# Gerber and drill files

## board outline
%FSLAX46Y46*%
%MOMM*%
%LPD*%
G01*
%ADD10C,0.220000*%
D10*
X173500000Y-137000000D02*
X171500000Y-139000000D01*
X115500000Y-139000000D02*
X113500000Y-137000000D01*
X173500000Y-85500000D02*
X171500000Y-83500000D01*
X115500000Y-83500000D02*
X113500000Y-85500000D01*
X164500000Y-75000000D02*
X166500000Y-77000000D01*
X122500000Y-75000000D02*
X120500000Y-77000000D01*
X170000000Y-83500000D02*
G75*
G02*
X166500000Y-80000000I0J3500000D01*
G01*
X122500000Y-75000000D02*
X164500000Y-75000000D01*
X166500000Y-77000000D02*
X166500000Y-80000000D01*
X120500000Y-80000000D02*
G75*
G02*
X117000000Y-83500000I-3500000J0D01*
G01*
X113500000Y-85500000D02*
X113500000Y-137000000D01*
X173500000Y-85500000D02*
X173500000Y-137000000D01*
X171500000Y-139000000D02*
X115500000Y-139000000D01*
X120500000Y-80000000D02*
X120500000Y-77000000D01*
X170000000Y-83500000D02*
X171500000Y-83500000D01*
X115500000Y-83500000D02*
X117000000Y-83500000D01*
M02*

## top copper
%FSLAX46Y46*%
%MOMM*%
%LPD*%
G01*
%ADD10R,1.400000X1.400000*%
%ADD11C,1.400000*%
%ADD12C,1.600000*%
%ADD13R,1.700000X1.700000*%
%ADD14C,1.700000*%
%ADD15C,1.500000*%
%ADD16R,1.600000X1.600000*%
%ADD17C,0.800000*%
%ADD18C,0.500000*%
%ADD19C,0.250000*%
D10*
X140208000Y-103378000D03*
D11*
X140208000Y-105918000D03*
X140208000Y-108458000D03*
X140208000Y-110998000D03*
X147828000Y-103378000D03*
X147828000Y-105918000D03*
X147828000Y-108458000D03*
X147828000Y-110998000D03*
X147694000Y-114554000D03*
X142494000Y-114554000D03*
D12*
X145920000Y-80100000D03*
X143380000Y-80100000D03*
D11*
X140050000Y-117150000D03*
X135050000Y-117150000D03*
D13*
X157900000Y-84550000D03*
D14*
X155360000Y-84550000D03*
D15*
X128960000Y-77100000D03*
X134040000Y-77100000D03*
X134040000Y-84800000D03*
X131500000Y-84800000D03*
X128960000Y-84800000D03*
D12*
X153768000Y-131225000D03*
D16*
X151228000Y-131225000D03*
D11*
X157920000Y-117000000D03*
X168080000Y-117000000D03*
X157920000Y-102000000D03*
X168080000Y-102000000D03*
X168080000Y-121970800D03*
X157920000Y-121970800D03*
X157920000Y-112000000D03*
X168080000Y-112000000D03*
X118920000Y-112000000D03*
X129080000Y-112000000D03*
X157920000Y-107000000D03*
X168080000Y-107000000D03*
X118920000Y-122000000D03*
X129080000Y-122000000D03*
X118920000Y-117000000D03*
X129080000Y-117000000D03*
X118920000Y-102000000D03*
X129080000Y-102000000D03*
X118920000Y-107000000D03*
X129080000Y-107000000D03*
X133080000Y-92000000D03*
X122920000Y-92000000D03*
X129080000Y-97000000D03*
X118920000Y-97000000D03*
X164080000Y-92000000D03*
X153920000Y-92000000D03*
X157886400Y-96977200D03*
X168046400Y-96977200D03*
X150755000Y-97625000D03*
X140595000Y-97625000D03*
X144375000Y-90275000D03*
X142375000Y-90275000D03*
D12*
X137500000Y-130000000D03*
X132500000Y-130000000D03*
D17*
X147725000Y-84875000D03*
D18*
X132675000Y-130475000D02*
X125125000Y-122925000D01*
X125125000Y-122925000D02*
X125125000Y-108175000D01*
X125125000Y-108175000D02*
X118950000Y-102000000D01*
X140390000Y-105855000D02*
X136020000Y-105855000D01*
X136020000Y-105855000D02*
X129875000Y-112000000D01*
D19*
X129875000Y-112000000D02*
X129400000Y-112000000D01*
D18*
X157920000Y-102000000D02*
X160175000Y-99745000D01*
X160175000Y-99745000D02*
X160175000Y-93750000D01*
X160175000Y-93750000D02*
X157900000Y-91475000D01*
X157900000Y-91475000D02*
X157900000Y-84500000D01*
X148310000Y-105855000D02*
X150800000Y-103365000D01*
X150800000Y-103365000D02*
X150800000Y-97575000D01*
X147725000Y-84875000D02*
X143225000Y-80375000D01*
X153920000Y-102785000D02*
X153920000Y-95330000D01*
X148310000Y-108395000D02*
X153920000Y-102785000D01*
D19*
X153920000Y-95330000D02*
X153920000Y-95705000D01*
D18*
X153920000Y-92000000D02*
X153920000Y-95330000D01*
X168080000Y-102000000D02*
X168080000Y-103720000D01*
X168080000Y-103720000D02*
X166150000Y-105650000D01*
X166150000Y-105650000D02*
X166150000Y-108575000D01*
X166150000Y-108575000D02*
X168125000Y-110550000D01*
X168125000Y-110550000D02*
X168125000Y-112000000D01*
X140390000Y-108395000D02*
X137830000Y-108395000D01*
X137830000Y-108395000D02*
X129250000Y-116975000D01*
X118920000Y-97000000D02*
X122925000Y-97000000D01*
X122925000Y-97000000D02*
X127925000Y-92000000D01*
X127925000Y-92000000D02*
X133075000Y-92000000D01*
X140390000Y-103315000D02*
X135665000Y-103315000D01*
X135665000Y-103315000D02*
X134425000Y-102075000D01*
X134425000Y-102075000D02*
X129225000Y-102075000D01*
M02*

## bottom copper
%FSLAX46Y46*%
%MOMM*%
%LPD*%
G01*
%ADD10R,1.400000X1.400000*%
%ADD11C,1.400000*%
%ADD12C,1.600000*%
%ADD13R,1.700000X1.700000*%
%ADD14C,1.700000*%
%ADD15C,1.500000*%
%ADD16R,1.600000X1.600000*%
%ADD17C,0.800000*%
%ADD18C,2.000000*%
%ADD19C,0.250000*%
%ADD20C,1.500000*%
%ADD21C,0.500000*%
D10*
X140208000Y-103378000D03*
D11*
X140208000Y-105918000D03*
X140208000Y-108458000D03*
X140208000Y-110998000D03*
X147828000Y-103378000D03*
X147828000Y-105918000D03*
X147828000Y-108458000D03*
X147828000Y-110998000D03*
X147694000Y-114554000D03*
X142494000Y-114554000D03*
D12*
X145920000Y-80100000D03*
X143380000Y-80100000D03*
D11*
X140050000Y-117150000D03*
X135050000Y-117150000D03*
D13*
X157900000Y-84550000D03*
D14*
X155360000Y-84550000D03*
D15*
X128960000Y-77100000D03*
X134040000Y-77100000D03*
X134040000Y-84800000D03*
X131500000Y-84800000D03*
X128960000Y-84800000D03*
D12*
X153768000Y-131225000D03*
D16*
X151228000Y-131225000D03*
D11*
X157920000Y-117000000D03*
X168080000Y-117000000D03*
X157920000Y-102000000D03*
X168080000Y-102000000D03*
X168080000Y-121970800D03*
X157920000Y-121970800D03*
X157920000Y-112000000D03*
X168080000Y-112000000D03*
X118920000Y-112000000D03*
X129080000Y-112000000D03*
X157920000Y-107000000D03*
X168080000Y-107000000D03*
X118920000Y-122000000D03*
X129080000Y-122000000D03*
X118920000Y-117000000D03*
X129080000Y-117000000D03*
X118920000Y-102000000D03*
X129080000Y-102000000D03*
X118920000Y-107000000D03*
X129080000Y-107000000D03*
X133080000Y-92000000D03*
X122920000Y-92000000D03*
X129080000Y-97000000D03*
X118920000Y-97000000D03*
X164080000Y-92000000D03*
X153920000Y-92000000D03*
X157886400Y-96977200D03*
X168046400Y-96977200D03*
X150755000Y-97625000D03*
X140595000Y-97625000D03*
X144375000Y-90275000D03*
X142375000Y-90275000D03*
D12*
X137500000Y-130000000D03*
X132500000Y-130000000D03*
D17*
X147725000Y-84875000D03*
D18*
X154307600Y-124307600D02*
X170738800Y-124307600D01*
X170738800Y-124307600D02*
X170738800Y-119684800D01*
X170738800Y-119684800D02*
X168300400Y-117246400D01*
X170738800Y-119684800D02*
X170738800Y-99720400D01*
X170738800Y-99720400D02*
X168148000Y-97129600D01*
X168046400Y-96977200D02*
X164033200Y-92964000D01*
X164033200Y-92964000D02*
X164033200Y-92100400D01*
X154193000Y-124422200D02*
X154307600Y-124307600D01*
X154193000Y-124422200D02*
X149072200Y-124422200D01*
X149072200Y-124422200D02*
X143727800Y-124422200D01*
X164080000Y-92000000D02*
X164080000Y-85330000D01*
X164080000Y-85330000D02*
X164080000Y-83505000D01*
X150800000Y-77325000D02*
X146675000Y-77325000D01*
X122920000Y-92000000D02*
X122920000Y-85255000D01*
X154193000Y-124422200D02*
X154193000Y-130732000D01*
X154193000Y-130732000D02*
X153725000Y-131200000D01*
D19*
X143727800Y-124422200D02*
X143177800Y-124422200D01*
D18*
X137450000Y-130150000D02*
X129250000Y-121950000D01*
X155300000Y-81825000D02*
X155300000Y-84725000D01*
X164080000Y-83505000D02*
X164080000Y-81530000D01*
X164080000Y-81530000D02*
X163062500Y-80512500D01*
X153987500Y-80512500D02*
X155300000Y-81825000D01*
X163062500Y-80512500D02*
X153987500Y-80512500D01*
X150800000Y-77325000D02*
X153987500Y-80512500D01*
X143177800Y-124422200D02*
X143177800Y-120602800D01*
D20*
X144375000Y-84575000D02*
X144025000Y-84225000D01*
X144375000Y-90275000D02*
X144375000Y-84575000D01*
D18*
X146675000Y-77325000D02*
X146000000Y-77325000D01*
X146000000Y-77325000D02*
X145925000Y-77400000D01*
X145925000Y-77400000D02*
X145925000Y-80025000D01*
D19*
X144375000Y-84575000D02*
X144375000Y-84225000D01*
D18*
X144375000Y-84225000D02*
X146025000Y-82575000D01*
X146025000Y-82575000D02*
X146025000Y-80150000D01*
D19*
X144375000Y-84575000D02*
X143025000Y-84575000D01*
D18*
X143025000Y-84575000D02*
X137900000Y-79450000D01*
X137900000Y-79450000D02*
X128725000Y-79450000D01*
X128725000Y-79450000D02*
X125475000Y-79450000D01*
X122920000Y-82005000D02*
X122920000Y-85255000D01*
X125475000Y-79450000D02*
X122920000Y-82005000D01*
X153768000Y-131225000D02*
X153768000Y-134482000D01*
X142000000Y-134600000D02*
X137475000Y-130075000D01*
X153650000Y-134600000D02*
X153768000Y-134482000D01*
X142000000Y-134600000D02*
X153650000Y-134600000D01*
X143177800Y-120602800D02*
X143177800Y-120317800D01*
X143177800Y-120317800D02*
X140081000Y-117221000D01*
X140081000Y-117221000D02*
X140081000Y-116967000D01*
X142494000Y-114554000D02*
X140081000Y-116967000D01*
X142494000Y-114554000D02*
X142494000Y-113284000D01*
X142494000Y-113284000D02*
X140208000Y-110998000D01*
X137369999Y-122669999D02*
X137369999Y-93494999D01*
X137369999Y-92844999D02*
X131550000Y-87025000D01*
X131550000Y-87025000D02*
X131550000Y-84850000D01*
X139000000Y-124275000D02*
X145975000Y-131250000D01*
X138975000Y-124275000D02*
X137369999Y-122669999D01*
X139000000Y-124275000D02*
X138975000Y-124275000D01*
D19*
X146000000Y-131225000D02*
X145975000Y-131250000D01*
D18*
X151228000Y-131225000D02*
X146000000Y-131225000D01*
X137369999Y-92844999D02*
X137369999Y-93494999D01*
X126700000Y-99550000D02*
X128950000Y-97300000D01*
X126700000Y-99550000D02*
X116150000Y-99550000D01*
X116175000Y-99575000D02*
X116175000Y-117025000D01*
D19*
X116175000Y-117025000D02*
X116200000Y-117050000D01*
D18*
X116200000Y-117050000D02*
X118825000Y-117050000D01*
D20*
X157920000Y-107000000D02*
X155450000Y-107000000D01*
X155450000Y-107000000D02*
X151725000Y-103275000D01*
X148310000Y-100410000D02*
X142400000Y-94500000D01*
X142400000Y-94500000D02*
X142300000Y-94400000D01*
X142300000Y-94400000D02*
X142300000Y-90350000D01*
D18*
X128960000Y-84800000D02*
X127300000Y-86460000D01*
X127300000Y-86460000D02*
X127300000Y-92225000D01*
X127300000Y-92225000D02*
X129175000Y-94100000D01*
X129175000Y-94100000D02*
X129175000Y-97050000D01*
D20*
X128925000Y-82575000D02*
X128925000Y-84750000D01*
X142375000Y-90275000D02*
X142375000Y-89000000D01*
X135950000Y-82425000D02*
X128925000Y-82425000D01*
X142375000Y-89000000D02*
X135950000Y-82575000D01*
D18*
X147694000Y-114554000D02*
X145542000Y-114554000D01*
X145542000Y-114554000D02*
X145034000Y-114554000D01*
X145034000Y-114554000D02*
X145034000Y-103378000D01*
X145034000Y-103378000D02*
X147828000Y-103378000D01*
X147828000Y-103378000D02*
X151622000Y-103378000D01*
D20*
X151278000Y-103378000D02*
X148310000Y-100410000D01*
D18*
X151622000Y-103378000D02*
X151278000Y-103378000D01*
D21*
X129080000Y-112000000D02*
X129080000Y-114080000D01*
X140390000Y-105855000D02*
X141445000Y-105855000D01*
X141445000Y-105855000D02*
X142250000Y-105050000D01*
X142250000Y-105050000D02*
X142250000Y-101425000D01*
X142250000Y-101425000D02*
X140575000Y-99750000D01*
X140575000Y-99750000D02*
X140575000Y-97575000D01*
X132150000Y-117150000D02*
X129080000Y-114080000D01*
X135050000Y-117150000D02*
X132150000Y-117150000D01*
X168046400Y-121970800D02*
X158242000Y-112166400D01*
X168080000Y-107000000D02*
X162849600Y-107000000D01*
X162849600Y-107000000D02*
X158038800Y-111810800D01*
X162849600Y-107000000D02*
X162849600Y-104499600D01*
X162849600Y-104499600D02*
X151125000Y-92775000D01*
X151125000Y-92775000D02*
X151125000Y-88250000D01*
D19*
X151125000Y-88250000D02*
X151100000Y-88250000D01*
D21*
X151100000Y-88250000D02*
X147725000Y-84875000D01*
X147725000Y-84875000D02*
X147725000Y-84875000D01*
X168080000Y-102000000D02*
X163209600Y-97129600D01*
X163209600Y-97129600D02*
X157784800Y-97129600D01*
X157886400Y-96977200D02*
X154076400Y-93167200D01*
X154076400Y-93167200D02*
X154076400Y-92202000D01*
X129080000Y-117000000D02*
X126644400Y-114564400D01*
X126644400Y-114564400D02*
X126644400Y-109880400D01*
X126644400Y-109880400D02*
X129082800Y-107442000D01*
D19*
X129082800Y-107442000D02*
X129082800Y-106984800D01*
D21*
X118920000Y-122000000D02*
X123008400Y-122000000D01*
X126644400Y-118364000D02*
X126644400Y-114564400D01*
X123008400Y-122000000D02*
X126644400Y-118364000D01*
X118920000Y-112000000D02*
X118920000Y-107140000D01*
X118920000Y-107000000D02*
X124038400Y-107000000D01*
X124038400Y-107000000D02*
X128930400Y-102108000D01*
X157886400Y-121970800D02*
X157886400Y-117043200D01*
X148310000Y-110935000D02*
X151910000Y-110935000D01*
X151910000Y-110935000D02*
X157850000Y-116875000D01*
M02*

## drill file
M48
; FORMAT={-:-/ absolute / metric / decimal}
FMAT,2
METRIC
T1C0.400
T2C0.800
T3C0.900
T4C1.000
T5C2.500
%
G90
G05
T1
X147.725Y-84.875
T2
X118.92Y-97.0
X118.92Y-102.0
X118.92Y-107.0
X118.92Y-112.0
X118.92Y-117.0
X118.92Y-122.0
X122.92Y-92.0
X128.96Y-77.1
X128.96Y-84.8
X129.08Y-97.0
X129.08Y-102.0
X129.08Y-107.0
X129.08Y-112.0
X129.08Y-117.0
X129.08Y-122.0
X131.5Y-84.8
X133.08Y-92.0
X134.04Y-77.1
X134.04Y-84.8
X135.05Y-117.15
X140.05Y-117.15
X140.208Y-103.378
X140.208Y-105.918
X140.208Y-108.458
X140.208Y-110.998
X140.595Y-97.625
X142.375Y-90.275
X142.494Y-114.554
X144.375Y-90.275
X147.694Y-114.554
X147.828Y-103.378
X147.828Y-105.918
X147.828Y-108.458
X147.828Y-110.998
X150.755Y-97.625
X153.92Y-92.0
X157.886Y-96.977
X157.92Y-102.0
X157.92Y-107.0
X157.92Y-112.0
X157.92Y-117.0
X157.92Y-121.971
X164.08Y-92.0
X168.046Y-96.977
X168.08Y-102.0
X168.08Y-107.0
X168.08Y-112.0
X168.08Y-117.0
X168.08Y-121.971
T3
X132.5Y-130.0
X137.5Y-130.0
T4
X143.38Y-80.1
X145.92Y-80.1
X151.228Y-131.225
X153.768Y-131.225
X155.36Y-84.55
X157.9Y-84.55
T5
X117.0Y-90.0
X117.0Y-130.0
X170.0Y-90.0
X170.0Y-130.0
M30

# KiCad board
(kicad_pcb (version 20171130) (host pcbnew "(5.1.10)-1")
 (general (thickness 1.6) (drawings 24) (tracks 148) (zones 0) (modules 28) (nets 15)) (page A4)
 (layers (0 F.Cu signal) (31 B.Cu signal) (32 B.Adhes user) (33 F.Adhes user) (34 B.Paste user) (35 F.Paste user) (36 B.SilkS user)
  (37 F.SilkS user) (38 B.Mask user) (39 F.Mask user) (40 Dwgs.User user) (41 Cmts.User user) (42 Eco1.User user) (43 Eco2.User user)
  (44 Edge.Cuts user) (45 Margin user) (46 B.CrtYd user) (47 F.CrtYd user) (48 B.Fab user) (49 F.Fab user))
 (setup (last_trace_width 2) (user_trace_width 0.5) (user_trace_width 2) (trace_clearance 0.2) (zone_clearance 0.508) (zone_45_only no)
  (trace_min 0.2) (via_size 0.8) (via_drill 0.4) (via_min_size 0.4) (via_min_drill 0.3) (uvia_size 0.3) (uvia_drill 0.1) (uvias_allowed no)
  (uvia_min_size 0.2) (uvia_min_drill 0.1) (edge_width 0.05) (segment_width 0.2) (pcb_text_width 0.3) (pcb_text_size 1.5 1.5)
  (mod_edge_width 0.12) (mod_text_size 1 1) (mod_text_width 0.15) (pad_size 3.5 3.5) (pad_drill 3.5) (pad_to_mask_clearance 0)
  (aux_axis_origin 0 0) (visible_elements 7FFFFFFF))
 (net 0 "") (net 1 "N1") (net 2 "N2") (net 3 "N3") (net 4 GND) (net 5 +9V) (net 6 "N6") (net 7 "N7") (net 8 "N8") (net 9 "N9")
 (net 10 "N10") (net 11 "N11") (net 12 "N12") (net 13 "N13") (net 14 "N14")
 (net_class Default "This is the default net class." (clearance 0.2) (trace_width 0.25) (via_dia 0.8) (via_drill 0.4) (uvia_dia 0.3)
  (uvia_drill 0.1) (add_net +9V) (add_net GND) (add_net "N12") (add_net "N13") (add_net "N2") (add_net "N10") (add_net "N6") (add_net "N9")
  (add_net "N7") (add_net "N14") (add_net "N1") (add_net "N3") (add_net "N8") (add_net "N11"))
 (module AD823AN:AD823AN (layer F.Cu) (at 144.018 107.188 270)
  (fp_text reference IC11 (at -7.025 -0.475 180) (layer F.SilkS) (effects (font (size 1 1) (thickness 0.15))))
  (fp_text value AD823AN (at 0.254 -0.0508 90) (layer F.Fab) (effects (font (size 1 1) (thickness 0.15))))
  (pad 1 thru_hole rect (at -3.81 3.81 270) (size 1.4 1.4) (drill 0.8) (layers *.Cu *.Mask) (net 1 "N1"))
  (pad 2 thru_hole circle (at -1.27 3.81 270) (size 1.4 1.4) (drill 0.8) (layers *.Cu *.Mask) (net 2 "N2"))
  (pad 3 thru_hole circle (at 1.27 3.81 270) (size 1.4 1.4) (drill 0.8) (layers *.Cu *.Mask) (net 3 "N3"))
  (pad 4 thru_hole circle (at 3.81 3.81 270) (size 1.4 1.4) (drill 0.8) (layers *.Cu *.Mask) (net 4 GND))
  (pad 8 thru_hole circle (at -3.81 -3.81 270) (size 1.4 1.4) (drill 0.8) (layers *.Cu *.Mask) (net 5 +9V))
  (pad 7 thru_hole circle (at -1.27 -3.81 270) (size 1.4 1.4) (drill 0.8) (layers *.Cu *.Mask) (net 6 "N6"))
  (pad 6 thru_hole circle (at 1.27 -3.81 270) (size 1.4 1.4) (drill 0.8) (layers *.Cu *.Mask) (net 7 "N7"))
  (pad 5 thru_hole circle (at 3.81 -3.81 270) (size 1.4 1.4) (drill 0.8) (layers *.Cu *.Mask) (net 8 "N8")))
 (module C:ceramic (layer F.Cu) (at 145.094 114.554)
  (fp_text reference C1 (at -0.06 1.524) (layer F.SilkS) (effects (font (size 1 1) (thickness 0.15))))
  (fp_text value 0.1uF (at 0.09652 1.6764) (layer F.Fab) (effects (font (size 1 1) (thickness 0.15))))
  (pad 2 thru_hole circle (at 2.6 0) (size 1.4 1.4) (drill 0.8) (layers *.Cu *.Mask) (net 5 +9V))
  (pad 1 thru_hole circle (at -2.6 0) (size 1.4 1.4) (drill 0.8) (layers *.Cu *.Mask) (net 4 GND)))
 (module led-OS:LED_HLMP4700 (layer F.Cu) (at 144.65 80.1)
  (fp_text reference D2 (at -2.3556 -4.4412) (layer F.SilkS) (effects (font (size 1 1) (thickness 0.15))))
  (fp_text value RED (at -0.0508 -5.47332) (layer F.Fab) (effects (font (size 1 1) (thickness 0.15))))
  (pad 2 thru_hole circle (at 1.27 0 90) (size 1.6 1.6) (drill 1) (layers *.Cu *.Mask) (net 4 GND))
  (pad 1 thru_hole circle (at -1.27 0 90) (size 1.6 1.6) (drill 1) (layers *.Cu *.Mask) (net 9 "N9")))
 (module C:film (layer F.Cu) (at 137.55 117.15)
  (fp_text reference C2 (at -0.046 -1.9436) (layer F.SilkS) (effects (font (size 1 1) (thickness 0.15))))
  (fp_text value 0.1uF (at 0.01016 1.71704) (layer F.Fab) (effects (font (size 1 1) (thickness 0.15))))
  (pad 2 thru_hole circle (at 2.5 0) (size 1.4 1.4) (drill 0.8) (layers *.Cu *.Mask) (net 4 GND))
  (pad 1 thru_hole circle (at -2.5 0) (size 1.4 1.4) (drill 0.8) (layers *.Cu *.Mask) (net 2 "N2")))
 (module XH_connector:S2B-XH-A (layer F.Cu) (at 157.9 84.55 180)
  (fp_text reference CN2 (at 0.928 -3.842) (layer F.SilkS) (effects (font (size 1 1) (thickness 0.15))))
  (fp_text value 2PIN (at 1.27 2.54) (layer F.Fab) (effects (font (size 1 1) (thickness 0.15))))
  (pad 1 thru_hole rect (at 0 0 180) (size 1.7 1.7) (drill 1) (layers *.Cu *.Mask) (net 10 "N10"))
  (pad 2 thru_hole circle (at 2.54 0 180) (size 1.7 1.7) (drill 1) (layers *.Cu *.Mask) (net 4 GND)))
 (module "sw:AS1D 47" (layer F.Cu) (at 131.5 79.8)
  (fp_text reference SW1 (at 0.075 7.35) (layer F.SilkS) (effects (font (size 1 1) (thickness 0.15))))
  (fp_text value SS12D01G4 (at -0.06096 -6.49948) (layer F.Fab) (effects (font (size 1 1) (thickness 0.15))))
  (pad 4 thru_hole circle (at -2.54 -2.7) (size 1.5 1.5) (drill 0.8) (layers *.Cu *.Mask))
  (pad 5 thru_hole circle (at 2.54 -2.7) (size 1.5 1.5) (drill 0.8) (layers *.Cu *.Mask))
  (pad 3 thru_hole circle (at 2.54 5) (size 1.5 1.5) (drill 0.8) (layers *.Cu *.Mask) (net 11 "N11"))
  (pad 2 thru_hole circle (at 0 5) (size 1.5 1.5) (drill 0.8) (layers *.Cu *.Mask) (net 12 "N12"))
  (pad 1 thru_hole circle (at -2.54 5) (size 1.5 1.5) (drill 0.8) (layers *.Cu *.Mask) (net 5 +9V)))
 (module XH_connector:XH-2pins (layer F.Cu) (at 152.625 131.225 90)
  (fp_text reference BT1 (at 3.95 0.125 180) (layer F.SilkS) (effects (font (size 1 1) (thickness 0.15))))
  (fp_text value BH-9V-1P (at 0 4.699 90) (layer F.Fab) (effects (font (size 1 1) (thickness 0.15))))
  (pad 2 thru_hole circle (at 0 1.143 90) (size 1.6 1.6) (drill 1) (layers *.Cu *.Mask) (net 4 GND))
  (pad 1 thru_hole rect (at 0 -1.397 90) (size 1.6 1.6) (drill 1) (layers *.Cu *.Mask) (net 12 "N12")))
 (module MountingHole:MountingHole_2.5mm (layer F.Cu) (at 170 130)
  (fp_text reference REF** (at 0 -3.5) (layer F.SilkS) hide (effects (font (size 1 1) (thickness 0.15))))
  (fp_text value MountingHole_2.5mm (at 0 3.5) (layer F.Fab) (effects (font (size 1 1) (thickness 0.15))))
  (pad 1 np_thru_hole circle (at 0 0) (size 2.5 2.5) (drill 2.5) (layers *.Cu *.Mask)))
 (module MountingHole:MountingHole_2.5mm (layer F.Cu) (at 117 130)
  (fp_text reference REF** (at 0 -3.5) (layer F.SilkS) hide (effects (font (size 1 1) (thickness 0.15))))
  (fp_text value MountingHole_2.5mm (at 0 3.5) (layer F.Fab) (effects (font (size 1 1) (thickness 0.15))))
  (pad 1 np_thru_hole circle (at 0 0) (size 2.5 2.5) (drill 2.5) (layers *.Cu *.Mask)))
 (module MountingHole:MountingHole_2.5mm (layer F.Cu) (at 170 90)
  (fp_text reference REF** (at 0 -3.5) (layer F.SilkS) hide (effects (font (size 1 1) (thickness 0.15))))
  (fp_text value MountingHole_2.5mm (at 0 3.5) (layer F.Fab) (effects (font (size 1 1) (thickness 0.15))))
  (pad 1 np_thru_hole circle (at 0 0) (size 2.5 2.5) (drill 2.5) (layers *.Cu *.Mask)))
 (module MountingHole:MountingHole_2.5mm (layer F.Cu) (at 117 90)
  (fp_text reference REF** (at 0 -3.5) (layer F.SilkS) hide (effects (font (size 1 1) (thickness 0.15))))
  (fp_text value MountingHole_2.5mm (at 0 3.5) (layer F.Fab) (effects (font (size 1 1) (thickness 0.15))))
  (pad 1 np_thru_hole circle (at 0 0) (size 2.5 2.5) (drill 2.5) (layers *.Cu *.Mask)))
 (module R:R (layer F.Cu) (at 163 117)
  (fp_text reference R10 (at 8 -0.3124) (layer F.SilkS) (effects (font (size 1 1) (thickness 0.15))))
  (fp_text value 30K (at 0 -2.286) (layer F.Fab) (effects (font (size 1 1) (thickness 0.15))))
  (pad 1 thru_hole circle (at -5.08 0) (size 1.4 1.4) (drill 0.8) (layers *.Cu *.Mask) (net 8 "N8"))
  (pad 2 thru_hole circle (at 5.08 0) (size 1.4 1.4) (drill 0.8) (layers *.Cu *.Mask) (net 4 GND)))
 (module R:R (layer F.Cu) (at 163 102)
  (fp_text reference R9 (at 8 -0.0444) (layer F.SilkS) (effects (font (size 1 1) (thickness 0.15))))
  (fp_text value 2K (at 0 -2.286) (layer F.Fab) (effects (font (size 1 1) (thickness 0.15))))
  (pad 1 thru_hole circle (at -5.08 0) (size 1.4 1.4) (drill 0.8) (layers *.Cu *.Mask) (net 10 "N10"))
  (pad 2 thru_hole circle (at 5.08 0) (size 1.4 1.4) (drill 0.8) (layers *.Cu *.Mask) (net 7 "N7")))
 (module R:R (layer F.Cu) (at 163 121.9708 180)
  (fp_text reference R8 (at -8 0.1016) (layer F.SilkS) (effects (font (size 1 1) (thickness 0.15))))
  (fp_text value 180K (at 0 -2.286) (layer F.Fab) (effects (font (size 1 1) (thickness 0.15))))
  (pad 1 thru_hole circle (at -5.08 0 180) (size 1.4 1.4) (drill 0.8) (layers *.Cu *.Mask) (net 9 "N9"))
  (pad 2 thru_hole circle (at 5.08 0 180) (size 1.4 1.4) (drill 0.8) (layers *.Cu *.Mask) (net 8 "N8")))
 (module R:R (layer F.Cu) (at 163 112)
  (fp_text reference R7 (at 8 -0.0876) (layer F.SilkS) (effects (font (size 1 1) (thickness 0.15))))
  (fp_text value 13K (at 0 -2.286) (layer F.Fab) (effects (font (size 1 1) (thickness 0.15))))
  (pad 1 thru_hole circle (at -5.08 0) (size 1.4 1.4) (drill 0.8) (layers *.Cu *.Mask) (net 9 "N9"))
  (pad 2 thru_hole circle (at 5.08 0) (size 1.4 1.4) (drill 0.8) (layers *.Cu *.Mask) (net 7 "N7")))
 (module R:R (layer F.Cu) (at 124 112)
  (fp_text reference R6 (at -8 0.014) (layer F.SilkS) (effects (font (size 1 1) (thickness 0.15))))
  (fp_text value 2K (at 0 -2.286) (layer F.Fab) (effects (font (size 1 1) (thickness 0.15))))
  (pad 1 thru_hole circle (at -5.08 0) (size 1.4 1.4) (drill 0.8) (layers *.Cu *.Mask) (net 1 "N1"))
  (pad 2 thru_hole circle (at 5.08 0) (size 1.4 1.4) (drill 0.8) (layers *.Cu *.Mask) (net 2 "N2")))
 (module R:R (layer F.Cu) (at 163 107)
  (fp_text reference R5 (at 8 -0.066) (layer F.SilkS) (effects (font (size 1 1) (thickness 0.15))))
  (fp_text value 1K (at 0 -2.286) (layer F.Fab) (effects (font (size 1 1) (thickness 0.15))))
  (pad 1 thru_hole circle (at -5.08 0) (size 1.4 1.4) (drill 0.8) (layers *.Cu *.Mask) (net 5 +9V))
  (pad 2 thru_hole circle (at 5.08 0) (size 1.4 1.4) (drill 0.8) (layers *.Cu *.Mask) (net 9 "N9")))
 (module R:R (layer F.Cu) (at 124 122)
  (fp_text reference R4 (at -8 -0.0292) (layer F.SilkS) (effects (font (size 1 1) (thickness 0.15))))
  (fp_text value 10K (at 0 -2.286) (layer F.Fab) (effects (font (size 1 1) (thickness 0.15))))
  (pad 1 thru_hole circle (at -5.08 0) (size 1.4 1.4) (drill 0.8) (layers *.Cu *.Mask) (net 3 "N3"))
  (pad 2 thru_hole circle (at 5.08 0) (size 1.4 1.4) (drill 0.8) (layers *.Cu *.Mask) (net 4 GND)))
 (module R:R (layer F.Cu) (at 124 117)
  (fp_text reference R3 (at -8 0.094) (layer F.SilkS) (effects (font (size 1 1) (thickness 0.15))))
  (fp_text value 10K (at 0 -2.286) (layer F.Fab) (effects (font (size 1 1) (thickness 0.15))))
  (pad 1 thru_hole circle (at -5.08 0) (size 1.4 1.4) (drill 0.8) (layers *.Cu *.Mask) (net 5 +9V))
  (pad 2 thru_hole circle (at 5.08 0) (size 1.4 1.4) (drill 0.8) (layers *.Cu *.Mask) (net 3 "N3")))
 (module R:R (layer F.Cu) (at 124 102)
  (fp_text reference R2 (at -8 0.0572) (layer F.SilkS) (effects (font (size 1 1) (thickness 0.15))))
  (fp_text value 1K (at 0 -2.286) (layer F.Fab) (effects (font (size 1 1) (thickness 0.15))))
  (pad 1 thru_hole circle (at -5.08 0) (size 1.4 1.4) (drill 0.8) (layers *.Cu *.Mask) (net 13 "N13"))
  (pad 2 thru_hole circle (at 5.08 0) (size 1.4 1.4) (drill 0.8) (layers *.Cu *.Mask) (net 1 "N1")))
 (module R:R (layer F.Cu) (at 124 107)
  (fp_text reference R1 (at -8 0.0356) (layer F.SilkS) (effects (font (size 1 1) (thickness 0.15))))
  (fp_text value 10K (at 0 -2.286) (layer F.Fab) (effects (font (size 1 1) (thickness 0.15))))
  (pad 1 thru_hole circle (at -5.08 0) (size 1.4 1.4) (drill 0.8) (layers *.Cu *.Mask) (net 1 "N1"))
  (pad 2 thru_hole circle (at 5.08 0) (size 1.4 1.4) (drill 0.8) (layers *.Cu *.Mask) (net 3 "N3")))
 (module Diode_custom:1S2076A (layer F.Cu) (at 128 92)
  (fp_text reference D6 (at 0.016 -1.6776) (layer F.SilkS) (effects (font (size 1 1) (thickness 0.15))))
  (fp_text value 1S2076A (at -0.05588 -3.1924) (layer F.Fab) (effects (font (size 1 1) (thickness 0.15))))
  (pad 2 thru_hole circle (at 5.08 0) (size 1.4 1.4) (drill 0.8) (layers *.Cu *.Mask) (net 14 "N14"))
  (pad 1 thru_hole circle (at -5.08 0) (size 1.4 1.4) (drill 0.8) (layers *.Cu *.Mask) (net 4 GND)))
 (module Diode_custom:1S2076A (layer F.Cu) (at 124 97)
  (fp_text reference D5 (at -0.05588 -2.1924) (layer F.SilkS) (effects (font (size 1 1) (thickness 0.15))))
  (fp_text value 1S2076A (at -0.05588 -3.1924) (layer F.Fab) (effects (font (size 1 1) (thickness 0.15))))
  (pad 2 thru_hole circle (at 5.08 0) (size 1.4 1.4) (drill 0.8) (layers *.Cu *.Mask) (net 5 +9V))
  (pad 1 thru_hole circle (at -5.08 0) (size 1.4 1.4) (drill 0.8) (layers *.Cu *.Mask) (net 14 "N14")))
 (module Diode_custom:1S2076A (layer F.Cu) (at 159 92)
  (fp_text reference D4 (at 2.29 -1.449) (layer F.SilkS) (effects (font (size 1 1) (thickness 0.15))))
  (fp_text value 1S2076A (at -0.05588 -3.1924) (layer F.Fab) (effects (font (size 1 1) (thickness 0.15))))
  (pad 2 thru_hole circle (at 5.08 0) (size 1.4 1.4) (drill 0.8) (layers *.Cu *.Mask) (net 4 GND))
  (pad 1 thru_hole circle (at -5.08 0) (size 1.4 1.4) (drill 0.8) (layers *.Cu *.Mask) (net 7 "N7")))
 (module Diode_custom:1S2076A (layer F.Cu) (at 162.9664 96.9772 180)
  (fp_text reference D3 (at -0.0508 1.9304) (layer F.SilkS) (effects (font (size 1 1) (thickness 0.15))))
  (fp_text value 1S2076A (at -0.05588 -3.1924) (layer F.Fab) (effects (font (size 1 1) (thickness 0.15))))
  (pad 2 thru_hole circle (at 5.08 0 180) (size 1.4 1.4) (drill 0.8) (layers *.Cu *.Mask) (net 7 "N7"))
  (pad 1 thru_hole circle (at -5.08 0 180) (size 1.4 1.4) (drill 0.8) (layers *.Cu *.Mask) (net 4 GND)))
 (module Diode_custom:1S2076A (layer F.Cu) (at 145.675 97.625)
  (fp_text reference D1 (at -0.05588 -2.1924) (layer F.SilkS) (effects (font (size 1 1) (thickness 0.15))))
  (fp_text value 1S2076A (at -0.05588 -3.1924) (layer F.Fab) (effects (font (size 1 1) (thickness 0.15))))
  (pad 2 thru_hole circle (at 5.08 0) (size 1.4 1.4) (drill 0.8) (layers *.Cu *.Mask) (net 6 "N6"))
  (pad 1 thru_hole circle (at -5.08 0) (size 1.4 1.4) (drill 0.8) (layers *.Cu *.Mask) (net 2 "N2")))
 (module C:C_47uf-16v (layer F.Cu) (at 143.375 90.275)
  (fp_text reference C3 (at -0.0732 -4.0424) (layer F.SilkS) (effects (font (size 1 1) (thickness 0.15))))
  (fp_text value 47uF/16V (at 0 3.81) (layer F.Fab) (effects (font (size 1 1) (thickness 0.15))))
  (pad 2 thru_hole circle (at 1 0) (size 1.4 1.4) (drill 0.8) (layers *.Cu *.Mask) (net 4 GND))
  (pad 1 thru_hole circle (at -1 0) (size 1.4 1.4) (drill 0.8) (layers *.Cu *.Mask) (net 5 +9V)))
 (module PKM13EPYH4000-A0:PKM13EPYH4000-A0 (layer F.Cu) (at 135 130)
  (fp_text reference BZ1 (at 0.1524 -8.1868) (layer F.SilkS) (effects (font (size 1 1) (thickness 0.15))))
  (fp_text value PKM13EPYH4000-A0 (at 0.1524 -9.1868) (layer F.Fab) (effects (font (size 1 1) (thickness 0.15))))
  (pad 2 thru_hole circle (at 2.5 0) (size 1.6 1.6) (drill 0.9) (layers *.Cu *.Mask) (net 4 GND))
  (pad 1 thru_hole circle (at -2.5 0) (size 1.6 1.6) (drill 0.9) (layers *.Cu *.Mask) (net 13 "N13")))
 (gr_line (start 173.5 137) (end 171.5 139) (layer Edge.Cuts) (width 0.22))
 (gr_line (start 115.5 139) (end 113.5 137) (layer Edge.Cuts) (width 0.22))
 (gr_line (start 173.5 85.5) (end 171.5 83.5) (layer Edge.Cuts) (width 0.22))
 (gr_line (start 115.5 83.5) (end 113.5 85.5) (layer Edge.Cuts) (width 0.22))
 (gr_line (start 164.5 75) (end 166.5 77) (layer Edge.Cuts) (width 0.22))
 (gr_line (start 122.5 75) (end 120.5 77) (layer Edge.Cuts) (width 0.22))
 (gr_arc (start 170 80) (end 166.5 80) (angle -90) (layer Edge.Cuts) (width 0.22))
 (gr_line (start 122.5 75) (end 164.5 75) (layer Edge.Cuts) (width 0.22))
 (gr_line (start 166.5 77) (end 166.5 80) (layer Edge.Cuts) (width 0.22))
 (gr_arc (start 117 80) (end 117 83.5) (angle -90) (layer Edge.Cuts) (width 0.22))
 (gr_line (start 113.5 85.5) (end 113.5 137) (layer Edge.Cuts) (width 0.22))
 (gr_line (start 173.5 85.5) (end 173.5 137) (layer Edge.Cuts) (width 0.22))
 (gr_line (start 171.5 139) (end 115.5 139) (layer Edge.Cuts) (width 0.22))
 (gr_line (start 120.5 80) (end 120.5 77) (layer Edge.Cuts) (width 0.22))
 (gr_line (start 170 83.5) (end 171.5 83.5) (layer Edge.Cuts) (width 0.22))
 (gr_line (start 115.5 83.5) (end 117 83.5) (layer Edge.Cuts) (width 0.22))
 (segment (start 154.3076 124.3076) (end 170.7388 124.3076) (width 2) (layer B.Cu) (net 4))
 (segment (start 170.7388 124.3076) (end 170.7388 119.6848) (width 2) (layer B.Cu) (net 4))
 (segment (start 170.7388 119.6848) (end 168.3004 117.2464) (width 2) (layer B.Cu) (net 4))
 (segment (start 170.7388 119.6848) (end 170.7388 99.7204) (width 2) (layer B.Cu) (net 4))
 (segment (start 170.7388 99.7204) (end 168.148 97.1296) (width 2) (layer B.Cu) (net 4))
 (segment (start 168.0464 96.9772) (end 164.0332 92.964) (width 2) (layer B.Cu) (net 4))
 (segment (start 164.0332 92.964) (end 164.0332 92.1004) (width 2) (layer B.Cu) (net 4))
 (segment (start 154.193 124.4222) (end 154.3076 124.3076) (width 2) (layer B.Cu) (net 4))
 (segment (start 154.193 124.4222) (end 149.0722 124.4222) (width 2) (layer B.Cu) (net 4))
 (segment (start 149.0722 124.4222) (end 143.7278 124.4222) (width 2) (layer B.Cu) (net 4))
 (segment (start 164.08 92) (end 164.08 85.33) (width 2) (layer B.Cu) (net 4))
 (segment (start 164.08 85.33) (end 164.08 83.505) (width 2) (layer B.Cu) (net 4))
 (segment (start 150.8 77.325) (end 146.675 77.325) (width 2) (layer B.Cu) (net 4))
 (segment (start 122.92 92) (end 122.92 85.255) (width 2) (layer B.Cu) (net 4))
 (segment (start 154.193 124.4222) (end 154.193 130.732) (width 2) (layer B.Cu) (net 4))
 (segment (start 154.193 130.732) (end 153.725 131.2) (width 2) (layer B.Cu) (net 4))
 (segment (start 143.7278 124.4222) (end 143.1778 124.4222) (width 0.25) (layer B.Cu) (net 4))
 (segment (start 137.45 130.15) (end 129.25 121.95) (width 2) (layer B.Cu) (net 4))
 (segment (start 155.3 81.825) (end 155.3 84.725) (width 2) (layer B.Cu) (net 4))
 (segment (start 164.08 83.505) (end 164.08 81.53) (width 2) (layer B.Cu) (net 4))
 (segment (start 164.08 81.53) (end 163.0625 80.5125) (width 2) (layer B.Cu) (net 4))
 (segment (start 153.9875 80.5125) (end 155.3 81.825) (width 2) (layer B.Cu) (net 4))
 (segment (start 163.0625 80.5125) (end 153.9875 80.5125) (width 2) (layer B.Cu) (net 4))
 (segment (start 150.8 77.325) (end 153.9875 80.5125) (width 2) (layer B.Cu) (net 4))
 (segment (start 143.1778 124.4222) (end 143.1778 120.6028) (width 2) (layer B.Cu) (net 4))
 (segment (start 144.375 84.575) (end 144.025 84.225) (width 1.5) (layer B.Cu) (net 4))
 (segment (start 144.375 90.275) (end 144.375 84.575) (width 1.5) (layer B.Cu) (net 4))
 (segment (start 146.675 77.325) (end 146 77.325) (width 2) (layer B.Cu) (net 4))
 (segment (start 146 77.325) (end 145.925 77.4) (width 2) (layer B.Cu) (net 4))
 (segment (start 145.925 77.4) (end 145.925 80.025) (width 2) (layer B.Cu) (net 4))
 (segment (start 144.375 84.575) (end 144.375 84.225) (width 0.25) (layer B.Cu) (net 4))
 (segment (start 144.375 84.225) (end 146.025 82.575) (width 2) (layer B.Cu) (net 4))
 (segment (start 146.025 82.575) (end 146.025 80.15) (width 2) (layer B.Cu) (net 4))
 (segment (start 144.375 84.575) (end 143.025 84.575) (width 0.25) (layer B.Cu) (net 4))
 (segment (start 143.025 84.575) (end 137.9 79.45) (width 2) (layer B.Cu) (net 4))
 (segment (start 137.9 79.45) (end 128.725 79.45) (width 2) (layer B.Cu) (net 4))
 (segment (start 128.725 79.45) (end 125.475 79.45) (width 2) (layer B.Cu) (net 4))
 (segment (start 122.92 82.005) (end 122.92 85.255) (width 2) (layer B.Cu) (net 4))
 (segment (start 125.475 79.45) (end 122.92 82.005) (width 2) (layer B.Cu) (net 4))
 (segment (start 153.768 131.225) (end 153.768 134.482) (width 2) (layer B.Cu) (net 4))
 (segment (start 142 134.6) (end 137.475 130.075) (width 2) (layer B.Cu) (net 4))
 (segment (start 153.65 134.6) (end 153.768 134.482) (width 2) (layer B.Cu) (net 4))
 (segment (start 142 134.6) (end 153.65 134.6) (width 2) (layer B.Cu) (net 4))
 (segment (start 143.1778 120.6028) (end 143.1778 120.3178) (width 2) (layer B.Cu) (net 4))
 (segment (start 143.1778 120.3178) (end 140.081 117.221) (width 2) (layer B.Cu) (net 4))
 (segment (start 140.081 117.221) (end 140.081 116.967) (width 2) (layer B.Cu) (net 4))
 (segment (start 142.494 114.554) (end 140.081 116.967) (width 2) (layer B.Cu) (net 4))
 (segment (start 142.494 114.554) (end 142.494 113.284) (width 2) (layer B.Cu) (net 4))
 (segment (start 142.494 113.284) (end 140.208 110.998) (width 2) (layer B.Cu) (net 4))
 (segment (start 137.369999 122.669999) (end 137.369999 93.494999) (width 2) (layer B.Cu) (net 12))
 (segment (start 137.369999 92.844999) (end 131.55 87.025) (width 2) (layer B.Cu) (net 12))
 (segment (start 131.55 87.025) (end 131.55 84.85) (width 2) (layer B.Cu) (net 12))
 (segment (start 139 124.275) (end 145.975 131.25) (width 2) (layer B.Cu) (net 12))
 (segment (start 138.975 124.275) (end 137.369999 122.669999) (width 2) (layer B.Cu) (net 12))
 (segment (start 139 124.275) (end 138.975 124.275) (width 2) (layer B.Cu) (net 12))
 (segment (start 146 131.225) (end 145.975 131.25) (width 0.25) (layer B.Cu) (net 12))
 (segment (start 151.228 131.225) (end 146 131.225) (width 2) (layer B.Cu) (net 12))
 (segment (start 137.369999 92.844999) (end 137.369999 93.494999) (width 2) (layer B.Cu) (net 12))
 (segment (start 132.675 130.475) (end 125.125 122.925) (width 0.5) (layer F.Cu) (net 13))
 (segment (start 125.125 122.925) (end 125.125 108.175) (width 0.5) (layer F.Cu) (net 13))
 (segment (start 125.125 108.175) (end 118.95 102) (width 0.5) (layer F.Cu) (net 13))
 (segment (start 126.7 99.55) (end 128.95 97.3) (width 2) (layer B.Cu) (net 5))
 (segment (start 126.7 99.55) (end 116.15 99.55) (width 2) (layer B.Cu) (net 5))
 (segment (start 116.175 99.575) (end 116.175 117.025) (width 2) (layer B.Cu) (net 5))
 (segment (start 116.175 117.025) (end 116.2 117.05) (width 0.25) (layer B.Cu) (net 5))
 (segment (start 116.2 117.05) (end 118.825 117.05) (width 2) (layer B.Cu) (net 5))
 (segment (start 157.92 107) (end 155.45 107) (width 1.5) (layer B.Cu) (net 5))
 (segment (start 155.45 107) (end 151.725 103.275) (width 1.5) (layer B.Cu) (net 5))
 (segment (start 148.31 100.41) (end 142.4 94.5) (width 1.5) (layer B.Cu) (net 5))
 (segment (start 142.4 94.5) (end 142.3 94.4) (width 1.5) (layer B.Cu) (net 5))
 (segment (start 142.3 94.4) (end 142.3 90.35) (width 1.5) (layer B.Cu) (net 5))
 (segment (start 128.96 84.8) (end 127.3 86.46) (width 2) (layer B.Cu) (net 5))
 (segment (start 127.3 86.46) (end 127.3 92.225) (width 2) (layer B.Cu) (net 5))
 (segment (start 127.3 92.225) (end 129.175 94.1) (width 2) (layer B.Cu) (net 5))
 (segment (start 129.175 94.1) (end 129.175 97.05) (width 2) (layer B.Cu) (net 5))
 (segment (start 128.925 82.575) (end 128.925 84.75) (width 1.5) (layer B.Cu) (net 5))
 (segment (start 142.375 90.275) (end 142.375 89) (width 1.5) (layer B.Cu) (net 5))
 (segment (start 135.95 82.425) (end 128.925 82.425) (width 1.5) (layer B.Cu) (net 5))
 (segment (start 142.375 89) (end 135.95 82.575) (width 1.5) (layer B.Cu) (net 5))
 (segment (start 147.694 114.554) (end 145.542 114.554) (width 2) (layer B.Cu) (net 5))
 (segment (start 145.542 114.554) (end 145.034 114.554) (width 2) (layer B.Cu) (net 5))
 (segment (start 145.034 114.554) (end 145.034 103.378) (width 2) (layer B.Cu) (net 5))
 (segment (start 145.034 103.378) (end 147.828 103.378) (width 2) (layer B.Cu) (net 5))
 (segment (start 147.828 103.378) (end 151.622 103.378) (width 2) (layer B.Cu) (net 5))
 (segment (start 151.278 103.378) (end 148.31 100.41) (width 1.5) (layer B.Cu) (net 5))
 (segment (start 151.622 103.378) (end 151.278 103.378) (width 2) (layer B.Cu) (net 5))
 (segment (start 129.08 112) (end 129.08 114.08) (width 0.5) (layer B.Cu) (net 2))
 (segment (start 140.39 105.855) (end 141.445 105.855) (width 0.5) (layer B.Cu) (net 2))
 (segment (start 141.445 105.855) (end 142.25 105.05) (width 0.5) (layer B.Cu) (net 2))
 (segment (start 142.25 105.05) (end 142.25 101.425) (width 0.5) (layer B.Cu) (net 2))
 (segment (start 142.25 101.425) (end 140.575 99.75) (width 0.5) (layer B.Cu) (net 2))
 (segment (start 140.575 99.75) (end 140.575 97.575) (width 0.5) (layer B.Cu) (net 2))
 (segment (start 140.39 105.855) (end 136.02 105.855) (width 0.5) (layer F.Cu) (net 2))
 (segment (start 136.02 105.855) (end 129.875 112) (width 0.5) (layer F.Cu) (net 2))
 (segment (start 129.875 112) (end 129.4 112) (width 0.25) (layer F.Cu) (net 2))
 (segment (start 132.15 117.15) (end 129.08 114.08) (width 0.5) (layer B.Cu) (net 2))
 (segment (start 135.05 117.15) (end 132.15 117.15) (width 0.5) (layer B.Cu) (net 2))
 (segment (start 157.92 102) (end 160.175 99.745) (width 0.5) (layer F.Cu) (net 10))
 (segment (start 160.175 99.745) (end 160.175 93.75) (width 0.5) (layer F.Cu) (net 10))
 (segment (start 160.175 93.75) (end 157.9 91.475) (width 0.5) (layer F.Cu) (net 10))
 (segment (start 157.9 91.475) (end 157.9 84.5) (width 0.5) (layer F.Cu) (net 10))
 (segment (start 148.31 105.855) (end 150.8 103.365) (width 0.5) (layer F.Cu) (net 6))
 (segment (start 150.8 103.365) (end 150.8 97.575) (width 0.5) (layer F.Cu) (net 6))
 (segment (start 168.0464 121.9708) (end 158.242 112.1664) (width 0.5) (layer B.Cu) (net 9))
 (segment (start 168.08 107) (end 162.8496 107) (width 0.5) (layer B.Cu) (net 9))
 (segment (start 162.8496 107) (end 158.0388 111.8108) (width 0.5) (layer B.Cu) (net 9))
 (segment (start 162.8496 107) (end 162.8496 104.4996) (width 0.5) (layer B.Cu) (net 9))
 (segment (start 162.8496 104.4996) (end 151.125 92.775) (width 0.5) (layer B.Cu) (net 9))
 (segment (start 151.125 92.775) (end 151.125 88.25) (width 0.5) (layer B.Cu) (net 9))
 (segment (start 151.125 88.25) (end 151.1 88.25) (width 0.25) (layer B.Cu) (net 9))
 (segment (start 151.1 88.25) (end 147.725 84.875) (width 0.5) (layer B.Cu) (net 9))
 (segment (start 147.725 84.875) (end 147.725 84.875) (width 0.5) (layer B.Cu) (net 9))
 (via (at 147.725 84.875) (size 0.8) (drill 0.4) (layers F.Cu B.Cu) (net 9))
 (segment (start 147.725 84.875) (end 143.225 80.375) (width 0.5) (layer F.Cu) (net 9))
 (segment (start 168.08 102) (end 163.2096 97.1296) (width 0.5) (layer B.Cu) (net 7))
 (segment (start 163.2096 97.1296) (end 157.7848 97.1296) (width 0.5) (layer B.Cu) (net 7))
 (segment (start 157.8864 96.9772) (end 154.0764 93.1672) (width 0.5) (layer B.Cu) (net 7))
 (segment (start 154.0764 93.1672) (end 154.0764 92.202) (width 0.5) (layer B.Cu) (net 7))
 (segment (start 153.92 102.785) (end 153.92 95.33) (width 0.5) (layer F.Cu) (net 7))
 (segment (start 148.31 108.395) (end 153.92 102.785) (width 0.5) (layer F.Cu) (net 7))
 (segment (start 153.92 95.33) (end 153.92 95.705) (width 0.25) (layer F.Cu) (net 7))
 (segment (start 153.92 92) (end 153.92 95.33) (width 0.5) (layer F.Cu) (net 7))
 (segment (start 168.08 102) (end 168.08 103.72) (width 0.5) (layer F.Cu) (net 7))
 (segment (start 168.08 103.72) (end 166.15 105.65) (width 0.5) (layer F.Cu) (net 7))
 (segment (start 166.15 105.65) (end 166.15 108.575) (width 0.5) (layer F.Cu) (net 7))
 (segment (start 166.15 108.575) (end 168.125 110.55) (width 0.5) (layer F.Cu) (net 7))
 (segment (start 168.125 110.55) (end 168.125 112) (width 0.5) (layer F.Cu) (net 7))
 (segment (start 129.08 117) (end 126.6444 114.5644) (width 0.5) (layer B.Cu) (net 3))
 (segment (start 126.6444 114.5644) (end 126.6444 109.8804) (width 0.5) (layer B.Cu) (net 3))
 (segment (start 126.6444 109.8804) (end 129.0828 107.442) (width 0.5) (layer B.Cu) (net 3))
 (segment (start 129.0828 107.442) (end 129.0828 106.9848) (width 0.25) (layer B.Cu) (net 3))
 (segment (start 118.92 122) (end 123.0084 122) (width 0.5) (layer B.Cu) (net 3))
 (segment (start 126.6444 118.364) (end 126.6444 114.5644) (width 0.5) (layer B.Cu) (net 3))
 (segment (start 123.0084 122) (end 126.6444 118.364) (width 0.5) (layer B.Cu) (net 3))
 (segment (start 140.39 108.395) (end 137.83 108.395) (width 0.5) (layer F.Cu) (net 3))
 (segment (start 137.83 108.395) (end 129.25 116.975) (width 0.5) (layer F.Cu) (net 3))
 (segment (start 118.92 97) (end 122.925 97) (width 0.5) (layer F.Cu) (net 14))
 (segment (start 122.925 97) (end 127.925 92) (width 0.5) (layer F.Cu) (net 14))
 (segment (start 127.925 92) (end 133.075 92) (width 0.5) (layer F.Cu) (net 14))
 (segment (start 118.92 112) (end 118.92 107.14) (width 0.5) (layer B.Cu) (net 1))
 (segment (start 118.92 107) (end 124.0384 107) (width 0.5) (layer B.Cu) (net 1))
 (segment (start 124.0384 107) (end 128.9304 102.108) (width 0.5) (layer B.Cu) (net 1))
 (segment (start 140.39 103.315) (end 135.665 103.315) (width 0.5) (layer F.Cu) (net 1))
 (segment (start 135.665 103.315) (end 134.425 102.075) (width 0.5) (layer F.Cu) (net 1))
 (segment (start 134.425 102.075) (end 129.225 102.075) (width 0.5) (layer F.Cu) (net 1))
 (segment (start 157.8864 121.9708) (end 157.8864 117.0432) (width 0.5) (layer B.Cu) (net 8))
 (segment (start 148.31 110.935) (end 151.91 110.935) (width 0.5) (layer B.Cu) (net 8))
 (segment (start 151.91 110.935) (end 157.85 116.875) (width 0.5) (layer B.Cu) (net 8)))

